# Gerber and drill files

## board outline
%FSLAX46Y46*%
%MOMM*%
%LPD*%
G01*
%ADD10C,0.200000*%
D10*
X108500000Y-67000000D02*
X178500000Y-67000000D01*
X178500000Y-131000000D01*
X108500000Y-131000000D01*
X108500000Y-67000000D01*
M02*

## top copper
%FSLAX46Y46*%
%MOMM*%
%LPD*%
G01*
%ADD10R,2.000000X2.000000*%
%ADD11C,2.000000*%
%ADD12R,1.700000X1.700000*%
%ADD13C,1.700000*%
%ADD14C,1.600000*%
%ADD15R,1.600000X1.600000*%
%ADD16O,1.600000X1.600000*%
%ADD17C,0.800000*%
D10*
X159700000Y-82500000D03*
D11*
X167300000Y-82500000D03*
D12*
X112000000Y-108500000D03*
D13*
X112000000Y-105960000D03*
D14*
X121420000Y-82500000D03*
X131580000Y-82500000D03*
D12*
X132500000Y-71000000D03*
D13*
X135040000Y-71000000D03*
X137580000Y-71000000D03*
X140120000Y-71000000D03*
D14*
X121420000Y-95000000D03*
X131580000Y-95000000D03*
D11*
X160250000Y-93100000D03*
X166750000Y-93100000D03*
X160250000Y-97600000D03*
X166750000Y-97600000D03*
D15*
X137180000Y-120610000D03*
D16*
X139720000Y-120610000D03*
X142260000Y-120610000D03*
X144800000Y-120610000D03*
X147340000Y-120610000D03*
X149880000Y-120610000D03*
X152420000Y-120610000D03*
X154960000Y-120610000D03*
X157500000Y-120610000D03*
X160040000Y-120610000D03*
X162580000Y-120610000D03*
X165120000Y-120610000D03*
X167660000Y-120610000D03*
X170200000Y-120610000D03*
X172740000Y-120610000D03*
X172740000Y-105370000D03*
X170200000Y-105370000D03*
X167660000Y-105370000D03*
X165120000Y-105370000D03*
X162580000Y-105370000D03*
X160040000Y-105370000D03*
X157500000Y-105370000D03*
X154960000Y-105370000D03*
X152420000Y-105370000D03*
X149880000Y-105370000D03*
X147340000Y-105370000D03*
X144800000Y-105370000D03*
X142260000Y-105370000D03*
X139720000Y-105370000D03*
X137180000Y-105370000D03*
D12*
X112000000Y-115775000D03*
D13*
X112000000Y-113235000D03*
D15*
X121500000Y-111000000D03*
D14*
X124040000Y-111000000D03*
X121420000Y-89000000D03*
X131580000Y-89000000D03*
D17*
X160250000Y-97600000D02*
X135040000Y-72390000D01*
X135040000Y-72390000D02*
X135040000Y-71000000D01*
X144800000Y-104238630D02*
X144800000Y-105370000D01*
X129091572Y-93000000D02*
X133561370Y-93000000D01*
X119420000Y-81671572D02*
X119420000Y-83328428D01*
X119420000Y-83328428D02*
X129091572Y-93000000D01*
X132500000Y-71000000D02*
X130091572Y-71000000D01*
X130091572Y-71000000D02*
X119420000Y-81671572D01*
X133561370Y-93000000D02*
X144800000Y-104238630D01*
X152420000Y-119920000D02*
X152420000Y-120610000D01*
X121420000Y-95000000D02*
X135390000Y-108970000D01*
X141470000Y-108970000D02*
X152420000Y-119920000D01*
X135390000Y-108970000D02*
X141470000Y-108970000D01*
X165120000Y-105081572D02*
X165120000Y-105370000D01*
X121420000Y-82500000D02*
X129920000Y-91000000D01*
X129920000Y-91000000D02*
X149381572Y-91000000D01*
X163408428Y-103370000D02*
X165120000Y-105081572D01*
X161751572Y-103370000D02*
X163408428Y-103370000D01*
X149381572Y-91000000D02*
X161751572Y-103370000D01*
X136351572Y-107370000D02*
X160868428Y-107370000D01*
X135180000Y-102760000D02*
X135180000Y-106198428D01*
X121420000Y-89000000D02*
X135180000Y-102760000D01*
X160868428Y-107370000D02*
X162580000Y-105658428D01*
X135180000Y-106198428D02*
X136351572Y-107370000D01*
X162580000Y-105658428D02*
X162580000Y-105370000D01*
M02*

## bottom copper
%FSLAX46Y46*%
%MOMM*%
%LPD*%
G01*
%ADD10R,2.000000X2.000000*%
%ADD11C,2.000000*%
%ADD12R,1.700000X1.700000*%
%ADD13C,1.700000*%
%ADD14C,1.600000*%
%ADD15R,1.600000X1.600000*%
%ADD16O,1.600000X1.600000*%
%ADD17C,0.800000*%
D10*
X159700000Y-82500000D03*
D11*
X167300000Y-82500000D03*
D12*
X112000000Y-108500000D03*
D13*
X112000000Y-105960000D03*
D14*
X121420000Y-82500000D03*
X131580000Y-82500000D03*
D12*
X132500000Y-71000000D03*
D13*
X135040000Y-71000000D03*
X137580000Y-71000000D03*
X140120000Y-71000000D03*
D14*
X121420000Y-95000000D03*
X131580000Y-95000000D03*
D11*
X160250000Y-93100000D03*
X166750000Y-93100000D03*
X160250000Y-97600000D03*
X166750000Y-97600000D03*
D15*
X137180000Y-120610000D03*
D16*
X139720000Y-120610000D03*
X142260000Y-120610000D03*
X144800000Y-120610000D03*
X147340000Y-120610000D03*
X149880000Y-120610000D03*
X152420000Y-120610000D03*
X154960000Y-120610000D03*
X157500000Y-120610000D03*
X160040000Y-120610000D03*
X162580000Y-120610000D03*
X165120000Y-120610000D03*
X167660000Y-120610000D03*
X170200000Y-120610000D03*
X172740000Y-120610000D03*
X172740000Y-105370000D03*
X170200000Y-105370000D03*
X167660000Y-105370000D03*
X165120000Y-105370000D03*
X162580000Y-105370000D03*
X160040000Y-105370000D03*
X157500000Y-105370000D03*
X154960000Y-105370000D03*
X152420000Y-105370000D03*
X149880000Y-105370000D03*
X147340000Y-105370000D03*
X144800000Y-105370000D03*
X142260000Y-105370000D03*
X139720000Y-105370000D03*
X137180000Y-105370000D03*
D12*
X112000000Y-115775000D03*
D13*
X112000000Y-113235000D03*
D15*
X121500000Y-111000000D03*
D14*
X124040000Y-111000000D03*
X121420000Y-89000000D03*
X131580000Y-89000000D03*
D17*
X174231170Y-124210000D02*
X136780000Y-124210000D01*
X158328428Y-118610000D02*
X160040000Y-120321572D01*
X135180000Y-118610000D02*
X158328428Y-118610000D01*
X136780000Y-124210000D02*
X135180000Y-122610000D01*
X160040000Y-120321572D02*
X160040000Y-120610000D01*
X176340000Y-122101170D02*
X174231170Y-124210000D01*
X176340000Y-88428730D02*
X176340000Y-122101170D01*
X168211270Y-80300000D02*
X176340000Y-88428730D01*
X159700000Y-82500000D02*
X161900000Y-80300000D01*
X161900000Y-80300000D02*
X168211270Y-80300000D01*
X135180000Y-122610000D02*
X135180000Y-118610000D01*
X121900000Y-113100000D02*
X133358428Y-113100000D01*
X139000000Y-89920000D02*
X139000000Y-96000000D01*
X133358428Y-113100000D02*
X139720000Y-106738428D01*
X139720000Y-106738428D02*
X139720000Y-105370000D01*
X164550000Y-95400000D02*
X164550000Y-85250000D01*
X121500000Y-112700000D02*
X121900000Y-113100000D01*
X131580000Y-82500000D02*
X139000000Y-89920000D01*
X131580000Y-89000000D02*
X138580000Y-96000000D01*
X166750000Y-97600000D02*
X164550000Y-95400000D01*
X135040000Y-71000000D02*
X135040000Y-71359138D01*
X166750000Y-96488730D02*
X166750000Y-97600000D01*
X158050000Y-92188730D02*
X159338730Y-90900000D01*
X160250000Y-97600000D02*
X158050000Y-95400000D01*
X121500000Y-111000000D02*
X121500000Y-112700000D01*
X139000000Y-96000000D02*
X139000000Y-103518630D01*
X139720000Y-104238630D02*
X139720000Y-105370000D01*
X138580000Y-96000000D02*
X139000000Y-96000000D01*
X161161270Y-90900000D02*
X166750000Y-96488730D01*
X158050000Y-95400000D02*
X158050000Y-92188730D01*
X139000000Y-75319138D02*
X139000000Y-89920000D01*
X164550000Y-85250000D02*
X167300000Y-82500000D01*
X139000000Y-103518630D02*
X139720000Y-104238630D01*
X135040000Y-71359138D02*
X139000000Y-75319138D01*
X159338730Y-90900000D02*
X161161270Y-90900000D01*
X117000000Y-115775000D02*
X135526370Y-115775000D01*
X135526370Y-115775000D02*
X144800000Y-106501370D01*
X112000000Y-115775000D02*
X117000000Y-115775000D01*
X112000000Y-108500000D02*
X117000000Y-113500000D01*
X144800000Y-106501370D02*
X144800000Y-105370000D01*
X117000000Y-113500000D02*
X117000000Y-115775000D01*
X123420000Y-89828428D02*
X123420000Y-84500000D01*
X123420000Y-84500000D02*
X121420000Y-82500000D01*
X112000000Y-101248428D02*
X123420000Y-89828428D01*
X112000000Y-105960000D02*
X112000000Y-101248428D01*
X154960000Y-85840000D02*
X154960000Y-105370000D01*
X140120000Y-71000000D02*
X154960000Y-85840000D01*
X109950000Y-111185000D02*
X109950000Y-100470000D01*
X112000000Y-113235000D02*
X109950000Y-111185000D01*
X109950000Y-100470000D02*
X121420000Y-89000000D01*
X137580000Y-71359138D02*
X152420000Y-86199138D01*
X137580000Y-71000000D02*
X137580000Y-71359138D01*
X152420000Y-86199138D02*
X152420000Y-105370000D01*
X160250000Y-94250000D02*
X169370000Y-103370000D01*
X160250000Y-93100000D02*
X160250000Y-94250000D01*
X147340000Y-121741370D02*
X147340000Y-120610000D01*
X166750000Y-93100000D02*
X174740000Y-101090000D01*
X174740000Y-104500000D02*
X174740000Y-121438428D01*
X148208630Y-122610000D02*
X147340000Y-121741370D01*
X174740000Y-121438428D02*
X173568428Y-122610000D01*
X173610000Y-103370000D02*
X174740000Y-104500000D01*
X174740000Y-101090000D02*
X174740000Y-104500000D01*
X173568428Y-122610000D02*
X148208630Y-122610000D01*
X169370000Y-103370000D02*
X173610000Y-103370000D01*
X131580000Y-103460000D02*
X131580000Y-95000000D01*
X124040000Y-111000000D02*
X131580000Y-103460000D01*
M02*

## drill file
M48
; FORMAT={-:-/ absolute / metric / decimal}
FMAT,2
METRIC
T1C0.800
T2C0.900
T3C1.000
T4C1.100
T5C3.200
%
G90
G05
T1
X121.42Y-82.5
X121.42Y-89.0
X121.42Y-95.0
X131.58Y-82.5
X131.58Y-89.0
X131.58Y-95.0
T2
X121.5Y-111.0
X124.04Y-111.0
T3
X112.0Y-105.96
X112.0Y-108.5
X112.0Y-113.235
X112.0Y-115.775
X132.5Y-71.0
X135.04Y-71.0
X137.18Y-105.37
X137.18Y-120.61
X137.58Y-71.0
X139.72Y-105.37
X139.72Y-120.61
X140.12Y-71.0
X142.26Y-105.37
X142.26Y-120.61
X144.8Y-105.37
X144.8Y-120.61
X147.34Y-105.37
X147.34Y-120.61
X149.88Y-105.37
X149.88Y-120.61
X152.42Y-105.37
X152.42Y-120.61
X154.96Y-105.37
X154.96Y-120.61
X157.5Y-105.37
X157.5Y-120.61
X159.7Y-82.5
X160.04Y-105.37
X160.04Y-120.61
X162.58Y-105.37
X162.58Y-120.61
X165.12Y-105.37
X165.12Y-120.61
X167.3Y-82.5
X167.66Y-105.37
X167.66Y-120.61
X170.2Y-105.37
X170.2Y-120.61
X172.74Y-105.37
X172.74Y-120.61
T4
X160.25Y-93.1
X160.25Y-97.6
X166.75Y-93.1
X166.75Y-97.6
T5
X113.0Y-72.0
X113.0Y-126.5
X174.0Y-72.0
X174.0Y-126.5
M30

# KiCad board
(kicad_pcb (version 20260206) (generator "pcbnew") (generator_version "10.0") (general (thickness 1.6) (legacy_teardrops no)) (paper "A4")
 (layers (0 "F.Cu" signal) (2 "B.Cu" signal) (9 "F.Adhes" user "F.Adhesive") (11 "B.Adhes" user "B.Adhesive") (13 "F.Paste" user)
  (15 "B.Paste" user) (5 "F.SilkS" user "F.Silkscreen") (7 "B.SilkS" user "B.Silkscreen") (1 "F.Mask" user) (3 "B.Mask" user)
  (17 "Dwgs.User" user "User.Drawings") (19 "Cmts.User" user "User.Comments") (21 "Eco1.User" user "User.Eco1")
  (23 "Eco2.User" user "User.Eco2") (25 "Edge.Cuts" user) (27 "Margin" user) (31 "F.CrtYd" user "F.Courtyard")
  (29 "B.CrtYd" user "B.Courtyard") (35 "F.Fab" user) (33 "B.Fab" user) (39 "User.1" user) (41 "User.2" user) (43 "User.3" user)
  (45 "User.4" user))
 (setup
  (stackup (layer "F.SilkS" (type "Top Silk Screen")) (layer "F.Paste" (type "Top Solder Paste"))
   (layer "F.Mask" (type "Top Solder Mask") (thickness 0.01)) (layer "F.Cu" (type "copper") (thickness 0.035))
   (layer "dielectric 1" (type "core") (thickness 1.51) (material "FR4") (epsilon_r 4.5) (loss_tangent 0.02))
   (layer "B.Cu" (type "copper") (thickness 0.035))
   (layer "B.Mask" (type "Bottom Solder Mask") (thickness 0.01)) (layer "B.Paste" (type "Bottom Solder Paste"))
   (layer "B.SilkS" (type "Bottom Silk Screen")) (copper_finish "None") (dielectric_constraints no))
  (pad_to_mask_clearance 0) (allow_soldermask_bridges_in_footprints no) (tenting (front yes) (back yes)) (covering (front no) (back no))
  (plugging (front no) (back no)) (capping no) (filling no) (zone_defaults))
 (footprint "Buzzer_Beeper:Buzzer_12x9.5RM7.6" (layer "F.Cu") (at 159.7 82.5)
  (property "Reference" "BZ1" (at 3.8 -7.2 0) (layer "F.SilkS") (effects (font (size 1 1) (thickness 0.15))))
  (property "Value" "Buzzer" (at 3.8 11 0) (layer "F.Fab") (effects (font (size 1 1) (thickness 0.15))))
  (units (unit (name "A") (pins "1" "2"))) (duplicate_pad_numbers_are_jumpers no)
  (pad "1" thru_hole rect (at 0 0) (size 2 2) (drill 1) (layers "*.Cu" "*.Mask") (remove_unused_layers no) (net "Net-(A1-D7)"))
  (pad "2" thru_hole circle (at 7.6 0) (size 2 2) (drill 1) (layers "*.Cu" "*.Mask") (remove_unused_layers no) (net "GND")))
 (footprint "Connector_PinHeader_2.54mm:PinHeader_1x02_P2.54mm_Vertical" (layer "F.Cu") (at 112 108.5 180)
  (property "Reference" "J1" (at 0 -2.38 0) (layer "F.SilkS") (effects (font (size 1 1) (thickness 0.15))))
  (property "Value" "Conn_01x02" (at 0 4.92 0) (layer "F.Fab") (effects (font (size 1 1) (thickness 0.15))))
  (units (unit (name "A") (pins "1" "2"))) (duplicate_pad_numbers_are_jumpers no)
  (pad "1" thru_hole rect (at 0 0 180) (size 1.7 1.7) (drill 1) (layers "*.Cu" "*.Mask") (remove_unused_layers no) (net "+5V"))
  (pad "2" thru_hole circle (at 0 2.54 180) (size 1.7 1.7) (drill 1) (layers "*.Cu" "*.Mask") (remove_unused_layers no) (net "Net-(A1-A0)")))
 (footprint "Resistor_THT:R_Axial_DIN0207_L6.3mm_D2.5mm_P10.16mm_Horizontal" (layer "F.Cu") (at 121.42 82.5)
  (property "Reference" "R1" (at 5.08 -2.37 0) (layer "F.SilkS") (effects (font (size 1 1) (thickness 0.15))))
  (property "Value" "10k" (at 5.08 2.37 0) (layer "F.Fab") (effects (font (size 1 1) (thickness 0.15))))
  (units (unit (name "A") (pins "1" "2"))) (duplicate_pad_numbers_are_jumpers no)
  (pad "1" thru_hole circle (at 0 0) (size 1.6 1.6) (drill 0.8) (layers "*.Cu" "*.Mask") (remove_unused_layers no) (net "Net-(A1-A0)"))
  (pad "2" thru_hole circle (at 10.16 0) (size 1.6 1.6) (drill 0.8) (layers "*.Cu" "*.Mask") (remove_unused_layers no) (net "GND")))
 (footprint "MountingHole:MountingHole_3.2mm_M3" (layer "F.Cu") (at 174 126.5)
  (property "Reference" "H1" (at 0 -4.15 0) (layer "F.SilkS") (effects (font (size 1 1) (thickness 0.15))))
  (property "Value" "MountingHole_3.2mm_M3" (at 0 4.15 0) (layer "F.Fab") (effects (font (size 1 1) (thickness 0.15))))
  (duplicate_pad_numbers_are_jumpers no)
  (pad "" np_thru_hole circle (at 0 0) (size 3.2 3.2) (drill 3.2) (layers "*.Cu" "*.Mask")))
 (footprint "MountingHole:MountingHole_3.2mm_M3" (layer "F.Cu") (at 174 72)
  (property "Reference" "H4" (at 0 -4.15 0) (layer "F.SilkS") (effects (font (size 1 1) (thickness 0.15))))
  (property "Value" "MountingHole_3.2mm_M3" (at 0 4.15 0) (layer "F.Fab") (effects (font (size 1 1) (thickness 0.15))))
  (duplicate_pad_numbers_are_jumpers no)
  (pad "" np_thru_hole circle (at 0 0) (size 3.2 3.2) (drill 3.2) (layers "*.Cu" "*.Mask")))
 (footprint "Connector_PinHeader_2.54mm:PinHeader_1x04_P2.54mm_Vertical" (layer "F.Cu") (at 132.5 71 90)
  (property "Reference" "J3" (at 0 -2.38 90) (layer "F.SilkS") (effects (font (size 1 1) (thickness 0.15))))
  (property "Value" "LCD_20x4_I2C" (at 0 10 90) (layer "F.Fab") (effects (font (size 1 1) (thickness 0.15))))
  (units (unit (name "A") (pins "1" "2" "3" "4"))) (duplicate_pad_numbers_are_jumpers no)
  (pad "1" thru_hole rect (at 0 0 90) (size 1.7 1.7) (drill 1) (layers "*.Cu" "*.Mask") (remove_unused_layers no) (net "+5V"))
  (pad "2" thru_hole circle (at 0 2.54 90) (size 1.7 1.7) (drill 1) (layers "*.Cu" "*.Mask") (remove_unused_layers no) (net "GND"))
  (pad "3" thru_hole circle (at 0 5.08 90) (size 1.7 1.7) (drill 1) (layers "*.Cu" "*.Mask") (remove_unused_layers no) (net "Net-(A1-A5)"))
  (pad "4" thru_hole circle (at 0 7.62 90) (size 1.7 1.7) (drill 1) (layers "*.Cu" "*.Mask") (remove_unused_layers no) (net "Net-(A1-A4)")))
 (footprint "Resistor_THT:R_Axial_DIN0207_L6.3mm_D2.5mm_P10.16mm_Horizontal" (layer "F.Cu") (at 121.42 95)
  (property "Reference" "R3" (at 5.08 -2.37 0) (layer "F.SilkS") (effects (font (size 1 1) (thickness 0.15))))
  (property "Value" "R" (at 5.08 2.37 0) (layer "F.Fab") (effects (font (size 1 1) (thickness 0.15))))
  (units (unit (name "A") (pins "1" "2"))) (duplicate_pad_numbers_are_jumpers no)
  (pad "1" thru_hole circle (at 0 0) (size 1.6 1.6) (drill 0.8) (layers "*.Cu" "*.Mask") (remove_unused_layers no) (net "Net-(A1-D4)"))
  (pad "2" thru_hole circle (at 10.16 0) (size 1.6 1.6) (drill 0.8) (layers "*.Cu" "*.Mask") (remove_unused_layers no) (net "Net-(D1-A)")))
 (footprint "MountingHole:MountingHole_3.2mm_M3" (layer "F.Cu") (at 113 72)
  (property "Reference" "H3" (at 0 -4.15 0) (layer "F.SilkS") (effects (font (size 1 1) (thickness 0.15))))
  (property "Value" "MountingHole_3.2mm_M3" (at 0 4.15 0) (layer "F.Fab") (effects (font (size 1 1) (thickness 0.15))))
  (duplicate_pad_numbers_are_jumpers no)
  (pad "" np_thru_hole circle (at 0 0) (size 3.2 3.2) (drill 3.2) (layers "*.Cu" "*.Mask")))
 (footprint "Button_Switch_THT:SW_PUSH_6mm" (layer "F.Cu") (at 160.25 93.1)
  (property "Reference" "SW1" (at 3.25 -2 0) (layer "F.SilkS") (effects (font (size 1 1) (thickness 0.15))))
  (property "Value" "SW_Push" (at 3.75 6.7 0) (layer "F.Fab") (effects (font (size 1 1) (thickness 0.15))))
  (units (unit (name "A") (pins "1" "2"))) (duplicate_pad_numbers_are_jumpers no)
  (pad "1" thru_hole circle (at 0 0 90) (size 2 2) (drill 1.1) (layers "*.Cu" "*.Mask") (remove_unused_layers no) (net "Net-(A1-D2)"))
  (pad "1" thru_hole circle (at 6.5 0 90) (size 2 2) (drill 1.1) (layers "*.Cu" "*.Mask") (remove_unused_layers no) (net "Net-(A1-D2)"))
  (pad "2" thru_hole circle (at 0 4.5 90) (size 2 2) (drill 1.1) (layers "*.Cu" "*.Mask") (remove_unused_layers no) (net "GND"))
  (pad "2" thru_hole circle (at 6.5 4.5 90) (size 2 2) (drill 1.1) (layers "*.Cu" "*.Mask") (remove_unused_layers no) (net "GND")))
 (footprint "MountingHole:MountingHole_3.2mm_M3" (layer "F.Cu") (at 113 126.5)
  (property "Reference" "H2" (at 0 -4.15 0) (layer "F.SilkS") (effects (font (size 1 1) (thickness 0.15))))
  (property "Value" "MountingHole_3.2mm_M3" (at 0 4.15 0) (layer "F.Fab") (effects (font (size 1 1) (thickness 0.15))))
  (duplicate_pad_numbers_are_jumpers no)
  (pad "" np_thru_hole circle (at 0 0) (size 3.2 3.2) (drill 3.2) (layers "*.Cu" "*.Mask")))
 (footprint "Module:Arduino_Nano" (layer "F.Cu") (at 137.18 120.61 90)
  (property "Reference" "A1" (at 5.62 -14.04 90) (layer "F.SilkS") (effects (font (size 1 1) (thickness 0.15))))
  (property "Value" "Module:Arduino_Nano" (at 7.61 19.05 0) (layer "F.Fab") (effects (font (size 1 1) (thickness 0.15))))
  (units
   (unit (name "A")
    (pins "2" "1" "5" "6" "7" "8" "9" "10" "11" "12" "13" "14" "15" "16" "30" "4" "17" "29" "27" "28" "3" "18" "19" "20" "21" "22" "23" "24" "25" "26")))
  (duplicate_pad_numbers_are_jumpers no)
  (pad "1" thru_hole rect (at 0 0 90) (size 1.6 1.6) (drill 1) (layers "*.Cu" "*.Mask") (remove_unused_layers no)
   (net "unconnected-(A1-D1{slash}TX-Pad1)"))
  (pad "2" thru_hole oval (at 0 2.54 90) (size 1.6 1.6) (drill 1) (layers "*.Cu" "*.Mask") (remove_unused_layers no)
   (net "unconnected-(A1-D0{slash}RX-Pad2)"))
  (pad "3" thru_hole oval (at 0 5.08 90) (size 1.6 1.6) (drill 1) (layers "*.Cu" "*.Mask") (remove_unused_layers no)
   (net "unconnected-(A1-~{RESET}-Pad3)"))
  (pad "4" thru_hole oval (at 0 7.62 90) (size 1.6 1.6) (drill 1) (layers "*.Cu" "*.Mask") (remove_unused_layers no)
   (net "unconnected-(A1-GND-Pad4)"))
  (pad "5" thru_hole oval (at 0 10.16 90) (size 1.6 1.6) (drill 1) (layers "*.Cu" "*.Mask") (remove_unused_layers no) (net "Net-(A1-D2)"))
  (pad "6" thru_hole oval (at 0 12.7 90) (size 1.6 1.6) (drill 1) (layers "*.Cu" "*.Mask") (remove_unused_layers no)
   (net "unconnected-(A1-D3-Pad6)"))
  (pad "7" thru_hole oval (at 0 15.24 90) (size 1.6 1.6) (drill 1) (layers "*.Cu" "*.Mask") (remove_unused_layers no) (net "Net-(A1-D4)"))
  (pad "8" thru_hole oval (at 0 17.78 90) (size 1.6 1.6) (drill 1) (layers "*.Cu" "*.Mask") (remove_unused_layers no)
   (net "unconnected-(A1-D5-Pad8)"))
  (pad "9" thru_hole oval (at 0 20.32 90) (size 1.6 1.6) (drill 1) (layers "*.Cu" "*.Mask") (remove_unused_layers no)
   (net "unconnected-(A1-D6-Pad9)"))
  (pad "10" thru_hole oval (at 0 22.86 90) (size 1.6 1.6) (drill 1) (layers "*.Cu" "*.Mask") (remove_unused_layers no) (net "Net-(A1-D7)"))
  (pad "11" thru_hole oval (at 0 25.4 90) (size 1.6 1.6) (drill 1) (layers "*.Cu" "*.Mask") (remove_unused_layers no)
   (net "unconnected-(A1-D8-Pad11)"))
  (pad "12" thru_hole oval (at 0 27.94 90) (size 1.6 1.6) (drill 1) (layers "*.Cu" "*.Mask") (remove_unused_layers no)
   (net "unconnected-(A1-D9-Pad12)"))
  (pad "13" thru_hole oval (at 0 30.48 90) (size 1.6 1.6) (drill 1) (layers "*.Cu" "*.Mask") (remove_unused_layers no)
   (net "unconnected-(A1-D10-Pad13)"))
  (pad "14" thru_hole oval (at 0 33.02 90) (size 1.6 1.6) (drill 1) (layers "*.Cu" "*.Mask") (remove_unused_layers no)
   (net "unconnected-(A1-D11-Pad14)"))
  (pad "15" thru_hole oval (at 0 35.56 90) (size 1.6 1.6) (drill 1) (layers "*.Cu" "*.Mask") (remove_unused_layers no)
   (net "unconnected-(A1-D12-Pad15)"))
  (pad "16" thru_hole oval (at 15.24 35.56 90) (size 1.6 1.6) (drill 1) (layers "*.Cu" "*.Mask") (remove_unused_layers no)
   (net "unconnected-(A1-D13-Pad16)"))
  (pad "17" thru_hole oval (at 15.24 33.02 90) (size 1.6 1.6) (drill 1) (layers "*.Cu" "*.Mask") (remove_unused_layers no)
   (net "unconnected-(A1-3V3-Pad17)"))
  (pad "18" thru_hole oval (at 15.24 30.48 90) (size 1.6 1.6) (drill 1) (layers "*.Cu" "*.Mask") (remove_unused_layers no)
   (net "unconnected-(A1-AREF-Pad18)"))
  (pad "19" thru_hole oval (at 15.24 27.94 90) (size 1.6 1.6) (drill 1) (layers "*.Cu" "*.Mask") (remove_unused_layers no)
   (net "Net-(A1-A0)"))
  (pad "20" thru_hole oval (at 15.24 25.4 90) (size 1.6 1.6) (drill 1) (layers "*.Cu" "*.Mask") (remove_unused_layers no)
   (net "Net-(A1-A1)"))
  (pad "21" thru_hole oval (at 15.24 22.86 90) (size 1.6 1.6) (drill 1) (layers "*.Cu" "*.Mask") (remove_unused_layers no)
   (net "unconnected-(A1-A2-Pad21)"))
  (pad "22" thru_hole oval (at 15.24 20.32 90) (size 1.6 1.6) (drill 1) (layers "*.Cu" "*.Mask") (remove_unused_layers no)
   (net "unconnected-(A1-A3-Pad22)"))
  (pad "23" thru_hole oval (at 15.24 17.78 90) (size 1.6 1.6) (drill 1) (layers "*.Cu" "*.Mask") (remove_unused_layers no)
   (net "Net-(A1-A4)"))
  (pad "24" thru_hole oval (at 15.24 15.24 90) (size 1.6 1.6) (drill 1) (layers "*.Cu" "*.Mask") (remove_unused_layers no)
   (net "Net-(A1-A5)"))
  (pad "25" thru_hole oval (at 15.24 12.7 90) (size 1.6 1.6) (drill 1) (layers "*.Cu" "*.Mask") (remove_unused_layers no)
   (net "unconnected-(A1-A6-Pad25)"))
  (pad "26" thru_hole oval (at 15.24 10.16 90) (size 1.6 1.6) (drill 1) (layers "*.Cu" "*.Mask") (remove_unused_layers no)
   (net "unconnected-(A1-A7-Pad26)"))
  (pad "27" thru_hole oval (at 15.24 7.62 90) (size 1.6 1.6) (drill 1) (layers "*.Cu" "*.Mask") (remove_unused_layers no) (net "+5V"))
  (pad "28" thru_hole oval (at 15.24 5.08 90) (size 1.6 1.6) (drill 1) (layers "*.Cu" "*.Mask") (remove_unused_layers no)
   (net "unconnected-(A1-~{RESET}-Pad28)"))
  (pad "29" thru_hole oval (at 15.24 2.54 90) (size 1.6 1.6) (drill 1) (layers "*.Cu" "*.Mask") (remove_unused_layers no) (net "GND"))
  (pad "30" thru_hole oval (at 15.24 0 90) (size 1.6 1.6) (drill 1) (layers "*.Cu" "*.Mask") (remove_unused_layers no)
   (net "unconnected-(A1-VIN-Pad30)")))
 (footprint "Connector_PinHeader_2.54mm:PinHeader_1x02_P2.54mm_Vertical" (layer "F.Cu") (at 112 115.775 180)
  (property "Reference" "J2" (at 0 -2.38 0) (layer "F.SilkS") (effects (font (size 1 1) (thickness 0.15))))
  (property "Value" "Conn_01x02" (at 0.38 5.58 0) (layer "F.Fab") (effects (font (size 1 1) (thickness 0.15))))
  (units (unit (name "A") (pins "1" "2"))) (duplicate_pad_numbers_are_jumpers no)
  (pad "1" thru_hole rect (at 0 0 180) (size 1.7 1.7) (drill 1) (layers "*.Cu" "*.Mask") (remove_unused_layers no) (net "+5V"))
  (pad "2" thru_hole circle (at 0 2.54 180) (size 1.7 1.7) (drill 1) (layers "*.Cu" "*.Mask") (remove_unused_layers no) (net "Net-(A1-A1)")))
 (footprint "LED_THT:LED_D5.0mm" (layer "F.Cu") (at 121.5 111)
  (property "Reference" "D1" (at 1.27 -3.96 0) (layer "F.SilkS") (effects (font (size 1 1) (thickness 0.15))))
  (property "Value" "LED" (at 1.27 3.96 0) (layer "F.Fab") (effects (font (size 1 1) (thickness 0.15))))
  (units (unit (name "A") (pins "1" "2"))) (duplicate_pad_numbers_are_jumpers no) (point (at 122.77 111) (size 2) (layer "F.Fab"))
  (pad "1" thru_hole rect (at 0 0) (size 1.6 1.6) (drill 0.9) (layers "*.Cu" "*.Mask") (remove_unused_layers no) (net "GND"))
  (pad "2" thru_hole circle (at 2.54 0) (size 1.6 1.6) (drill 0.9) (layers "*.Cu" "*.Mask") (remove_unused_layers no) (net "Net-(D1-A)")))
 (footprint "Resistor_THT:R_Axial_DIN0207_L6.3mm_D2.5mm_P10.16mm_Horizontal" (layer "F.Cu") (at 121.42 89)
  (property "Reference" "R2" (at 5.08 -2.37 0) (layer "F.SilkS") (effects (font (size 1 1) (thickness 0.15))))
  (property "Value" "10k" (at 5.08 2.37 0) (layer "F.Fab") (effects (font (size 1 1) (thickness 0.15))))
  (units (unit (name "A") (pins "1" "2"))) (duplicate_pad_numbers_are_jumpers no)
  (pad "1" thru_hole circle (at 0 0) (size 1.6 1.6) (drill 0.8) (layers "*.Cu" "*.Mask") (remove_unused_layers no) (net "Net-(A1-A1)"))
  (pad "2" thru_hole circle (at 10.16 0) (size 1.6 1.6) (drill 0.8) (layers "*.Cu" "*.Mask") (remove_unused_layers no) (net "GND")))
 (gr_rect (start 108.5 67) (end 178.5 131) (stroke (width 0.2) (type solid)) (fill no) (layer "Edge.Cuts"))
 (segment (start 174.23117 124.21) (end 136.78 124.21) (width 0.8) (layer "B.Cu") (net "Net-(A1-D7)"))
 (segment (start 158.328428 118.61) (end 160.04 120.321572) (width 0.8) (layer "B.Cu") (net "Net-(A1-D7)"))
 (segment (start 135.18 118.61) (end 158.328428 118.61) (width 0.8) (layer "B.Cu") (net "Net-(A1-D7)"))
 (segment (start 136.78 124.21) (end 135.18 122.61) (width 0.8) (layer "B.Cu") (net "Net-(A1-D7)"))
 (segment (start 160.04 120.321572) (end 160.04 120.61) (width 0.8) (layer "B.Cu") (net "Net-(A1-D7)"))
 (segment (start 176.34 122.10117) (end 174.23117 124.21) (width 0.8) (layer "B.Cu") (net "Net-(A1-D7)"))
 (segment (start 176.34 88.42873) (end 176.34 122.10117) (width 0.8) (layer "B.Cu") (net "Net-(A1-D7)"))
 (segment (start 168.21127 80.3) (end 176.34 88.42873) (width 0.8) (layer "B.Cu") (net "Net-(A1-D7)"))
 (segment (start 159.7 82.5) (end 161.9 80.3) (width 0.8) (layer "B.Cu") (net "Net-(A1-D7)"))
 (segment (start 161.9 80.3) (end 168.21127 80.3) (width 0.8) (layer "B.Cu") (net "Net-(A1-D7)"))
 (segment (start 135.18 122.61) (end 135.18 118.61) (width 0.8) (layer "B.Cu") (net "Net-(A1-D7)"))
 (segment (start 160.25 97.6) (end 135.04 72.39) (width 0.8) (layer "F.Cu") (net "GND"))
 (segment (start 135.04 72.39) (end 135.04 71) (width 0.8) (layer "F.Cu") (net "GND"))
 (segment (start 121.9 113.1) (end 133.358428 113.1) (width 0.8) (layer "B.Cu") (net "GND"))
 (segment (start 139 89.92) (end 139 96) (width 0.8) (layer "B.Cu") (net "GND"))
 (segment (start 133.358428 113.1) (end 139.72 106.738428) (width 0.8) (layer "B.Cu") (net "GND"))
 (segment (start 139.72 106.738428) (end 139.72 105.37) (width 0.8) (layer "B.Cu") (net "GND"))
 (segment (start 164.55 95.4) (end 164.55 85.25) (width 0.8) (layer "B.Cu") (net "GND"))
 (segment (start 121.5 112.7) (end 121.9 113.1) (width 0.8) (layer "B.Cu") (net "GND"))
 (segment (start 131.58 82.5) (end 139 89.92) (width 0.8) (layer "B.Cu") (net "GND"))
 (segment (start 131.58 89) (end 138.58 96) (width 0.8) (layer "B.Cu") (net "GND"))
 (segment (start 166.75 97.6) (end 164.55 95.4) (width 0.8) (layer "B.Cu") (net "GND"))
 (segment (start 135.04 71) (end 135.04 71.359138) (width 0.8) (layer "B.Cu") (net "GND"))
 (segment (start 166.75 96.48873) (end 166.75 97.6) (width 0.8) (layer "B.Cu") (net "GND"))
 (segment (start 158.05 92.18873) (end 159.33873 90.9) (width 0.8) (layer "B.Cu") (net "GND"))
 (segment (start 160.25 97.6) (end 158.05 95.4) (width 0.8) (layer "B.Cu") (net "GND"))
 (segment (start 121.5 111) (end 121.5 112.7) (width 0.8) (layer "B.Cu") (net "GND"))
 (segment (start 139 96) (end 139 103.51863) (width 0.8) (layer "B.Cu") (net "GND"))
 (segment (start 139.72 104.23863) (end 139.72 105.37) (width 0.8) (layer "B.Cu") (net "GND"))
 (segment (start 138.58 96) (end 139 96) (width 0.8) (layer "B.Cu") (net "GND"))
 (segment (start 161.16127 90.9) (end 166.75 96.48873) (width 0.8) (layer "B.Cu") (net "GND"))
 (segment (start 158.05 95.4) (end 158.05 92.18873) (width 0.8) (layer "B.Cu") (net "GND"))
 (segment (start 139 75.319138) (end 139 89.92) (width 0.8) (layer "B.Cu") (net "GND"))
 (segment (start 164.55 85.25) (end 167.3 82.5) (width 0.8) (layer "B.Cu") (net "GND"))
 (segment (start 139 103.51863) (end 139.72 104.23863) (width 0.8) (layer "B.Cu") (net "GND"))
 (segment (start 135.04 71.359138) (end 139 75.319138) (width 0.8) (layer "B.Cu") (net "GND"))
 (segment (start 159.33873 90.9) (end 161.16127 90.9) (width 0.8) (layer "B.Cu") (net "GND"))
 (segment (start 144.8 104.23863) (end 144.8 105.37) (width 0.8) (layer "F.Cu") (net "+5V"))
 (segment (start 129.091572 93) (end 133.56137 93) (width 0.8) (layer "F.Cu") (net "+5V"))
 (segment (start 119.42 81.671572) (end 119.42 83.328428) (width 0.8) (layer "F.Cu") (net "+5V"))
 (segment (start 119.42 83.328428) (end 129.091572 93) (width 0.8) (layer "F.Cu") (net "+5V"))
 (segment (start 132.5 71) (end 130.091572 71) (width 0.8) (layer "F.Cu") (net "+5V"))
 (segment (start 130.091572 71) (end 119.42 81.671572) (width 0.8) (layer "F.Cu") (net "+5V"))
 (segment (start 133.56137 93) (end 144.8 104.23863) (width 0.8) (layer "F.Cu") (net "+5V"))
 (segment (start 117 115.775) (end 135.52637 115.775) (width 0.8) (layer "B.Cu") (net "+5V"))
 (segment (start 135.52637 115.775) (end 144.8 106.50137) (width 0.8) (layer "B.Cu") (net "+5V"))
 (segment (start 112 115.775) (end 117 115.775) (width 0.8) (layer "B.Cu") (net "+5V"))
 (segment (start 112 108.5) (end 117 113.5) (width 0.8) (layer "B.Cu") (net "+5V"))
 (segment (start 144.8 106.50137) (end 144.8 105.37) (width 0.8) (layer "B.Cu") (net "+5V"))
 (segment (start 117 113.5) (end 117 115.775) (width 0.8) (layer "B.Cu") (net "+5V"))
 (segment (start 152.42 119.92) (end 152.42 120.61) (width 0.8) (layer "F.Cu") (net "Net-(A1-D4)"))
 (segment (start 121.42 95) (end 135.39 108.97) (width 0.8) (layer "F.Cu") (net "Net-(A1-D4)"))
 (segment (start 141.47 108.97) (end 152.42 119.92) (width 0.8) (layer "F.Cu") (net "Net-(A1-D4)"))
 (segment (start 135.39 108.97) (end 141.47 108.97) (width 0.8) (layer "F.Cu") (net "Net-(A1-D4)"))
 (segment (start 165.12 105.081572) (end 165.12 105.37) (width 0.8) (layer "F.Cu") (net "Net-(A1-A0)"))
 (segment (start 121.42 82.5) (end 129.92 91) (width 0.8) (layer "F.Cu") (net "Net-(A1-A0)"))
 (segment (start 129.92 91) (end 149.381572 91) (width 0.8) (layer "F.Cu") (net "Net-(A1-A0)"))
 (segment (start 163.408428 103.37) (end 165.12 105.081572) (width 0.8) (layer "F.Cu") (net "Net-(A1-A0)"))
 (segment (start 161.751572 103.37) (end 163.408428 103.37) (width 0.8) (layer "F.Cu") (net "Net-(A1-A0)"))
 (segment (start 149.381572 91) (end 161.751572 103.37) (width 0.8) (layer "F.Cu") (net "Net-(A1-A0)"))
 (segment (start 123.42 89.828428) (end 123.42 84.5) (width 0.8) (layer "B.Cu") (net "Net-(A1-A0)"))
 (segment (start 123.42 84.5) (end 121.42 82.5) (width 0.8) (layer "B.Cu") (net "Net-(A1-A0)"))
 (segment (start 112 101.248428) (end 123.42 89.828428) (width 0.8) (layer "B.Cu") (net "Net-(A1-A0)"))
 (segment (start 112 105.96) (end 112 101.248428) (width 0.8) (layer "B.Cu") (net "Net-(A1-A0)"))
 (segment (start 154.96 85.84) (end 154.96 105.37) (width 0.8) (layer "B.Cu") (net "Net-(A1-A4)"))
 (segment (start 140.12 71) (end 154.96 85.84) (width 0.8) (layer "B.Cu") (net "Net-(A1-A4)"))
 (segment (start 136.351572 107.37) (end 160.868428 107.37) (width 0.8) (layer "F.Cu") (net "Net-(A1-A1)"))
 (segment (start 135.18 102.76) (end 135.18 106.198428) (width 0.8) (layer "F.Cu") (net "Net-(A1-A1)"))
 (segment (start 121.42 89) (end 135.18 102.76) (width 0.8) (layer "F.Cu") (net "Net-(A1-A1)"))
 (segment (start 160.868428 107.37) (end 162.58 105.658428) (width 0.8) (layer "F.Cu") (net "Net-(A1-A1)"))
 (segment (start 135.18 106.198428) (end 136.351572 107.37) (width 0.8) (layer "F.Cu") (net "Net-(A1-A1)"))
 (segment (start 162.58 105.658428) (end 162.58 105.37) (width 0.8) (layer "F.Cu") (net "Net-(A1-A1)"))
 (segment (start 109.95 111.185) (end 109.95 100.47) (width 0.8) (layer "B.Cu") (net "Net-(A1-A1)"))
 (segment (start 112 113.235) (end 109.95 111.185) (width 0.8) (layer "B.Cu") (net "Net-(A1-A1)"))
 (segment (start 109.95 100.47) (end 121.42 89) (width 0.8) (layer "B.Cu") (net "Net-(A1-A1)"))
 (segment (start 137.58 71.359138) (end 152.42 86.199138) (width 0.8) (layer "B.Cu") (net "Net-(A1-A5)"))
 (segment (start 137.58 71) (end 137.58 71.359138) (width 0.8) (layer "B.Cu") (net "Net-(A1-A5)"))
 (segment (start 152.42 86.199138) (end 152.42 105.37) (width 0.8) (layer "B.Cu") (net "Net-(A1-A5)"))
 (segment (start 160.25 94.25) (end 169.37 103.37) (width 0.8) (layer "B.Cu") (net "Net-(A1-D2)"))
 (segment (start 160.25 93.1) (end 160.25 94.25) (width 0.8) (layer "B.Cu") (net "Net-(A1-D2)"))
 (segment (start 147.34 121.74137) (end 147.34 120.61) (width 0.8) (layer "B.Cu") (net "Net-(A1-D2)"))
 (segment (start 166.75 93.1) (end 174.74 101.09) (width 0.8) (layer "B.Cu") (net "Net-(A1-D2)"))
 (segment (start 174.74 104.5) (end 174.74 121.438428) (width 0.8) (layer "B.Cu") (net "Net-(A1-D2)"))
 (segment (start 148.20863 122.61) (end 147.34 121.74137) (width 0.8) (layer "B.Cu") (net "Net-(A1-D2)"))
 (segment (start 174.74 121.438428) (end 173.568428 122.61) (width 0.8) (layer "B.Cu") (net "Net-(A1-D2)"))
 (segment (start 173.61 103.37) (end 174.74 104.5) (width 0.8) (layer "B.Cu") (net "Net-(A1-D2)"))
 (segment (start 174.74 101.09) (end 174.74 104.5) (width 0.8) (layer "B.Cu") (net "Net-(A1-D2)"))
 (segment (start 173.568428 122.61) (end 148.20863 122.61) (width 0.8) (layer "B.Cu") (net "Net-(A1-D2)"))
 (segment (start 169.37 103.37) (end 173.61 103.37) (width 0.8) (layer "B.Cu") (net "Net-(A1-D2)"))
 (segment (start 131.58 103.46) (end 131.58 95) (width 0.8) (layer "B.Cu") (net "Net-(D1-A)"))
 (segment (start 124.04 111) (end 131.58 103.46) (width 0.8) (layer "B.Cu") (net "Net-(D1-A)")))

